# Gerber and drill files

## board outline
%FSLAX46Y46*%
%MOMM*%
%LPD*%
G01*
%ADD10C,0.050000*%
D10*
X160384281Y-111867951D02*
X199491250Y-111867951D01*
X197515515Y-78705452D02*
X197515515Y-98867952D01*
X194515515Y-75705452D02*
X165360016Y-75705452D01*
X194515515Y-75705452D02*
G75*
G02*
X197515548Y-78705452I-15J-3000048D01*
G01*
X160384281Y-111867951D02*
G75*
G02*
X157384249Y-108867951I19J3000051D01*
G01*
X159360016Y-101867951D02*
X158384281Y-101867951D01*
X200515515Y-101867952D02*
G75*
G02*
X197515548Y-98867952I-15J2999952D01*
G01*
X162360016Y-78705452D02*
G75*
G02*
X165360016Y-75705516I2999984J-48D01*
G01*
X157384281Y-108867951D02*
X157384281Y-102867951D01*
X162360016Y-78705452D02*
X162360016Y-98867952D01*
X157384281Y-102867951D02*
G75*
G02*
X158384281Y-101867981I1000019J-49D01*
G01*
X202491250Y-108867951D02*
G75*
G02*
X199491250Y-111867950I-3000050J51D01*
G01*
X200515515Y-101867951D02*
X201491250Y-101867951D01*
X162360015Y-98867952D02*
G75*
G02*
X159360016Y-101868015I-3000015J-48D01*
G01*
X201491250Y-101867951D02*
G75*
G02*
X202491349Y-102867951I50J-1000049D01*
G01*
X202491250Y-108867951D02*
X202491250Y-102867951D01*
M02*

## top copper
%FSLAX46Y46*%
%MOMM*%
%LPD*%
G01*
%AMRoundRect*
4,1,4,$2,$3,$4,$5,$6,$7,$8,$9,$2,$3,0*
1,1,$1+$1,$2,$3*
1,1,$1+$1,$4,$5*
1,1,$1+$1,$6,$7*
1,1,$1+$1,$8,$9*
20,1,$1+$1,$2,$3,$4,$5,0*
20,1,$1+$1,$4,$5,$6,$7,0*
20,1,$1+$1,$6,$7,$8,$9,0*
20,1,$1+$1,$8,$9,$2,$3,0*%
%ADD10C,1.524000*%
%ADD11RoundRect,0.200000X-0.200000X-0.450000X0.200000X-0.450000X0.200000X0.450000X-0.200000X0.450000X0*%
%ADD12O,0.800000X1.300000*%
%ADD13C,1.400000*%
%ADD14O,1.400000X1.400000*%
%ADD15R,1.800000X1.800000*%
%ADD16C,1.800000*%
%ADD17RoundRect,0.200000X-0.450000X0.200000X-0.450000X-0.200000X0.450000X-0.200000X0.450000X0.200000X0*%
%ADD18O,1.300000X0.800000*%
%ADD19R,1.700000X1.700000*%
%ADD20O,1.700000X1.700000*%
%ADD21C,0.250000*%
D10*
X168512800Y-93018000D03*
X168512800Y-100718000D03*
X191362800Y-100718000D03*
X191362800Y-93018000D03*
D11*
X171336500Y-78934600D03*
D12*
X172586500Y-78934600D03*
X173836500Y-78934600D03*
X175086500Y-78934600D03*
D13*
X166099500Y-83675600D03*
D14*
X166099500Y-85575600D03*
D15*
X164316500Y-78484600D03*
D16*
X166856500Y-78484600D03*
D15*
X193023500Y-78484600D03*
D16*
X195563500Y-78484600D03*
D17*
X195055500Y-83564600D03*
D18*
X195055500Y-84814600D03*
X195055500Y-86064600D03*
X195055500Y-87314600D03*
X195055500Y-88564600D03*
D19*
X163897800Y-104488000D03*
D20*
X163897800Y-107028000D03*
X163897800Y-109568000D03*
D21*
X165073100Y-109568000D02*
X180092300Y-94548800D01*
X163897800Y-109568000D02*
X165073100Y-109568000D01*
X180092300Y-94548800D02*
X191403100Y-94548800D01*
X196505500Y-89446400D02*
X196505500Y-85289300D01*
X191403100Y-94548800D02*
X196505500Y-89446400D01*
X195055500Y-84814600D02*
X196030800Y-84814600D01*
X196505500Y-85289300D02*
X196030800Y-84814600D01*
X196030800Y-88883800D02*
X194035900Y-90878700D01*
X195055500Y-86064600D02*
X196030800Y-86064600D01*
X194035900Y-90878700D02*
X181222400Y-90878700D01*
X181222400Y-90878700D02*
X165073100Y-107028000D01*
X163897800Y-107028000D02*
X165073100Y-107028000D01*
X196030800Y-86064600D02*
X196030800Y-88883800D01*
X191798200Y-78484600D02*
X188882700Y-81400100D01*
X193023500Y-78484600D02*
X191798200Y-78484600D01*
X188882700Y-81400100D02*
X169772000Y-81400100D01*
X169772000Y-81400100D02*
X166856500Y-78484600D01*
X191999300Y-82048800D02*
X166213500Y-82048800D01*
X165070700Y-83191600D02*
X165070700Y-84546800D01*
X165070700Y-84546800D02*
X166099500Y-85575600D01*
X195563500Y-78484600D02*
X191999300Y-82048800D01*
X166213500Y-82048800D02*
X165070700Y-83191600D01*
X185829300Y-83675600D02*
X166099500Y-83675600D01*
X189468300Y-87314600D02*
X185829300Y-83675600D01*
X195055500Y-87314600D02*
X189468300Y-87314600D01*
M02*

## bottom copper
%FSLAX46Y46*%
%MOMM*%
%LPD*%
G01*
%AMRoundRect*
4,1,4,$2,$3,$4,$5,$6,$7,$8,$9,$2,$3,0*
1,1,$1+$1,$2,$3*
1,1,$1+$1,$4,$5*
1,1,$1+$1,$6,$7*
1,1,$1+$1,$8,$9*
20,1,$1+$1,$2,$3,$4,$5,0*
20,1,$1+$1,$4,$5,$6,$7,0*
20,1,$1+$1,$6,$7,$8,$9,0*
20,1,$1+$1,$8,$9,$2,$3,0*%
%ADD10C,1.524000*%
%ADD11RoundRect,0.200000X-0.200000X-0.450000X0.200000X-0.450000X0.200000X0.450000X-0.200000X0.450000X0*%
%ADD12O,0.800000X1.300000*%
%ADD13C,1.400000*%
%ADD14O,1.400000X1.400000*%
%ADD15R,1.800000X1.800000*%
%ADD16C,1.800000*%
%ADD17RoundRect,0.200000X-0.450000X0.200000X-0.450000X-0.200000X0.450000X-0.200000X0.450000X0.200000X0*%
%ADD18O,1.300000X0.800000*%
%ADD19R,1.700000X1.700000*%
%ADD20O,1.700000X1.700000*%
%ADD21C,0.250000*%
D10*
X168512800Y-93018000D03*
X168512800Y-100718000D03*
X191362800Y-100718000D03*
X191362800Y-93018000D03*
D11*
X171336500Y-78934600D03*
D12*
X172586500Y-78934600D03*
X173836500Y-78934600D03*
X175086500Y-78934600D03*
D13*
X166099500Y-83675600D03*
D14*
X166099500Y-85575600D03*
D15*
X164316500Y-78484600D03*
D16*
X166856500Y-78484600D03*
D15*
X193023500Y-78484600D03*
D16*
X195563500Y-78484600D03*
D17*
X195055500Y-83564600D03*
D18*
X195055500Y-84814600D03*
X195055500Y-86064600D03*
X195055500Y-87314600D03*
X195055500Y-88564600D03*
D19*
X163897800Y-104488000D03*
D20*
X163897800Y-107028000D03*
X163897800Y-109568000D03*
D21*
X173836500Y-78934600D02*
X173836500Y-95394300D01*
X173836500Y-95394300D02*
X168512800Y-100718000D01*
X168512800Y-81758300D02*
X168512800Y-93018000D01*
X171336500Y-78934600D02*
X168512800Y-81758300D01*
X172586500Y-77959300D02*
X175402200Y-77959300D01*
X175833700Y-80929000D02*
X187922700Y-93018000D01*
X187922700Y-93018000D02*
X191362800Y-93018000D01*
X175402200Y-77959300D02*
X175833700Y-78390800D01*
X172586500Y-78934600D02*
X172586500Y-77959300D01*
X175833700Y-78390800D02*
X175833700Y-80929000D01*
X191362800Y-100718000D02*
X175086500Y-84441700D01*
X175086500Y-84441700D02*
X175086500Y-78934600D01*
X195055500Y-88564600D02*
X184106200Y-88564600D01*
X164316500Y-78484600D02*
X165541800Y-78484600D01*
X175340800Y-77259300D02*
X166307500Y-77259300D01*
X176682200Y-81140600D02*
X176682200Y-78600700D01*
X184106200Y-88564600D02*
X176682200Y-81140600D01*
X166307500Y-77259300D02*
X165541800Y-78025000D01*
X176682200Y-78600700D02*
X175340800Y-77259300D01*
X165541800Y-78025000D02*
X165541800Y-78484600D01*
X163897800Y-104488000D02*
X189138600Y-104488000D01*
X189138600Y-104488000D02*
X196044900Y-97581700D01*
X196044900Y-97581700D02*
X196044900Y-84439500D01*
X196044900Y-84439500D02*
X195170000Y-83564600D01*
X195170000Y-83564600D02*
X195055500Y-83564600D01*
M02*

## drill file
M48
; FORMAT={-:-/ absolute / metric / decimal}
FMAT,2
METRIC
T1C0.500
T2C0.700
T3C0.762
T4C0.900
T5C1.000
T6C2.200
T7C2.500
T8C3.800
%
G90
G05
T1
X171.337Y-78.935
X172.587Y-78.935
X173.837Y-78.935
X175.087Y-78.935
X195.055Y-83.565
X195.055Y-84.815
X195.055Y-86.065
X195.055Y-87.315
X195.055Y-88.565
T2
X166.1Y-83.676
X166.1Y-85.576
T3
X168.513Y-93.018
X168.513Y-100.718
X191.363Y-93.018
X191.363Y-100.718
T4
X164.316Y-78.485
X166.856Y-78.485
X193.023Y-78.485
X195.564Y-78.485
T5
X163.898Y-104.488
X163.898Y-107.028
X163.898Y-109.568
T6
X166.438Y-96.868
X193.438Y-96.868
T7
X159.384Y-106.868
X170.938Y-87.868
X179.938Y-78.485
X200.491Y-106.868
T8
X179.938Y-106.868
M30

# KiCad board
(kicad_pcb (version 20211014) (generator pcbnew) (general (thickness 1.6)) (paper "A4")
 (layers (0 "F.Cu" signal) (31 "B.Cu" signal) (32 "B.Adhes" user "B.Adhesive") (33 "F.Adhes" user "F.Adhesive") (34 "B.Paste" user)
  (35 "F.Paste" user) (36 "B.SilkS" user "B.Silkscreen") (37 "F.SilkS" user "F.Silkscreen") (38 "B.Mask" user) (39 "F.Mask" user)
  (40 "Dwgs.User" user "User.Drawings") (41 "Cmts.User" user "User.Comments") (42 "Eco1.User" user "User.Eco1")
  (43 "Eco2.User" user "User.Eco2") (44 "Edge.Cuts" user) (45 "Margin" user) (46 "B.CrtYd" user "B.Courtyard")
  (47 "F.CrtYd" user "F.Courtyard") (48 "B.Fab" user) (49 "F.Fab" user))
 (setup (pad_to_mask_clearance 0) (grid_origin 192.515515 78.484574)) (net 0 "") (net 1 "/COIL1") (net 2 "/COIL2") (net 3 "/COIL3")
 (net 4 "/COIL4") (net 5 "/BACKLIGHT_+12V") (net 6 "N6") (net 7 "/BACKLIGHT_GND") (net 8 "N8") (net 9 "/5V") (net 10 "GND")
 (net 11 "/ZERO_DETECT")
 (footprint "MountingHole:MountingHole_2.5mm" (layer "F.Cu") (at 179.9378 78.4846)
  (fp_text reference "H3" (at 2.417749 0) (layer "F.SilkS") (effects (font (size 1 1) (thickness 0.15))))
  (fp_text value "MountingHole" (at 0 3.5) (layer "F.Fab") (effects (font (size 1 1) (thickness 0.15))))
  (pad "" np_thru_hole circle locked (at 0 0) (size 2.5 2.5) (drill 2.5) (layers *.Cu *.Mask)))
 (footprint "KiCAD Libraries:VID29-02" (layer "F.Cu") (at 180.1028 96.868)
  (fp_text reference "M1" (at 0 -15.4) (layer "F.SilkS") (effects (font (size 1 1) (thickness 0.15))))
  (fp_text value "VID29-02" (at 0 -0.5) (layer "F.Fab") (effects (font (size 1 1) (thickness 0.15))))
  (pad "" np_thru_hole circle locked (at -9.165 -9) (size 2.5 2.5) (drill 2.5) (layers *.Cu *.Mask))
  (pad "" np_thru_hole circle locked (at 13.335 0) (size 2.2 2.2) (drill 2.2) (layers *.Cu *.Mask))
  (pad "" np_thru_hole circle locked (at -0.165 10) (size 3.8 3.8) (drill 3.8) (layers *.Cu *.Mask))
  (pad "" np_thru_hole circle locked (at -13.665 0) (size 2.2 2.2) (drill 2.2) (layers *.Cu *.Mask))
  (pad "1" thru_hole circle locked (at -11.59 -3.85) (size 1.524 1.524) (drill 0.762) (layers *.Cu *.Mask) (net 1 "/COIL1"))
  (pad "2" thru_hole circle locked (at -11.59 3.85) (size 1.524 1.524) (drill 0.762) (layers *.Cu *.Mask) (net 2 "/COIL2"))
  (pad "3" thru_hole circle locked (at 11.26 3.85) (size 1.524 1.524) (drill 0.762) (layers *.Cu *.Mask) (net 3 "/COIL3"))
  (pad "4" thru_hole circle locked (at 11.26 -3.85) (size 1.524 1.524) (drill 0.762) (layers *.Cu *.Mask) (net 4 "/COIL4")))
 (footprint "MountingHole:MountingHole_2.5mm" (layer "F.Cu") (at 159.3843 106.868)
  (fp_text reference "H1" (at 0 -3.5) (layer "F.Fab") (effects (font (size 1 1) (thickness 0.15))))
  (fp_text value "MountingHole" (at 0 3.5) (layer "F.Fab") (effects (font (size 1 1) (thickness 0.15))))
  (pad "" np_thru_hole circle locked (at 0 0) (size 2.5 2.5) (drill 2.5) (layers *.Cu *.Mask)))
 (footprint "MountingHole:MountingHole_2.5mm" (layer "F.Cu") (at 200.4913 106.868)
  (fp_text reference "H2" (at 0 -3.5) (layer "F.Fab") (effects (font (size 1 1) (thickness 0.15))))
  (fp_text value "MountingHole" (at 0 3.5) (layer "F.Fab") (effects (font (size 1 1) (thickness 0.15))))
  (pad "" np_thru_hole circle locked (at 0 0) (size 2.5 2.5) (drill 2.5) (layers *.Cu *.Mask)))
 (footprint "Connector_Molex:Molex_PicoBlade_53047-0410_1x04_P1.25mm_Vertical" (layer "F.Cu") (at 171.3365 78.9346)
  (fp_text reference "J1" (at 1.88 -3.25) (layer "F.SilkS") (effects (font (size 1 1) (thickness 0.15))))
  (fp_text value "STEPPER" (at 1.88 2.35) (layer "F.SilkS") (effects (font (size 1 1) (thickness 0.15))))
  (pad "1" thru_hole roundrect (at 0 0) (size 0.8 1.3) (drill 0.5) (layers *.Cu *.Mask) (roundrect_rratio 0.25) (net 1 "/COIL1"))
  (pad "2" thru_hole oval (at 1.25 0) (size 0.8 1.3) (drill 0.5) (layers *.Cu *.Mask) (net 4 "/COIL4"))
  (pad "3" thru_hole oval (at 2.5 0) (size 0.8 1.3) (drill 0.5) (layers *.Cu *.Mask) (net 2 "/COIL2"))
  (pad "4" thru_hole oval (at 3.75 0) (size 0.8 1.3) (drill 0.5) (layers *.Cu *.Mask) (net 3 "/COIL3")))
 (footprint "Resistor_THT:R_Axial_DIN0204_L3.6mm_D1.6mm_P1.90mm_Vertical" (layer "F.Cu") (at 166.0995 83.6756 -90)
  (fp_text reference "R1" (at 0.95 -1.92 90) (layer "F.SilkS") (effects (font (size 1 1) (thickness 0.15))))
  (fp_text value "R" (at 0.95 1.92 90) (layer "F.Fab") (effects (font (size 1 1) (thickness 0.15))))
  (pad "1" thru_hole circle (at 0 0 270) (size 1.4 1.4) (drill 0.7) (layers *.Cu *.Mask) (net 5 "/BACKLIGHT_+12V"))
  (pad "2" thru_hole oval (at 1.9 0 270) (size 1.4 1.4) (drill 0.7) (layers *.Cu *.Mask) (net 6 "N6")))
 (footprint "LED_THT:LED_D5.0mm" (layer "F.Cu") (at 164.3165 78.4846)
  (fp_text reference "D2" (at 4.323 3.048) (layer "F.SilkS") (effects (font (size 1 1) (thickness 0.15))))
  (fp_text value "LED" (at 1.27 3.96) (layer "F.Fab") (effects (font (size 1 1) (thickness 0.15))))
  (pad "1" thru_hole rect (at 0 0) (size 1.8 1.8) (drill 0.9) (layers *.Cu *.Mask) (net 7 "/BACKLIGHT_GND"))
  (pad "2" thru_hole circle (at 2.54 0) (size 1.8 1.8) (drill 0.9) (layers *.Cu *.Mask) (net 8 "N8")))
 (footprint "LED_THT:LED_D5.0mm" (layer "F.Cu") (at 193.0235 78.4846)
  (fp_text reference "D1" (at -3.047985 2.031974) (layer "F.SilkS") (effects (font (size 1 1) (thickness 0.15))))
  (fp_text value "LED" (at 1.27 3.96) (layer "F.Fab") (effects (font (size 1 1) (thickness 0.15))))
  (pad "1" thru_hole rect (at 0 0) (size 1.8 1.8) (drill 0.9) (layers *.Cu *.Mask) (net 8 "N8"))
  (pad "2" thru_hole circle (at 2.54 0) (size 1.8 1.8) (drill 0.9) (layers *.Cu *.Mask) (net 6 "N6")))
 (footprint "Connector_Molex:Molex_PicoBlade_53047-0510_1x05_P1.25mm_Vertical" (layer "F.Cu") (at 195.0555 83.5646 -90)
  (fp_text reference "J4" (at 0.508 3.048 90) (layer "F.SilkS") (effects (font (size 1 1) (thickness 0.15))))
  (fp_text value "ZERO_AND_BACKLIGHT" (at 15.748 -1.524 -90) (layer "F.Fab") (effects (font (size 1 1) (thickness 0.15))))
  (pad "1" thru_hole roundrect (at 0 0 270) (size 0.8 1.3) (drill 0.5) (layers *.Cu *.Mask) (roundrect_rratio 0.25) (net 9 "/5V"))
  (pad "2" thru_hole oval (at 1.25 0 270) (size 0.8 1.3) (drill 0.5) (layers *.Cu *.Mask) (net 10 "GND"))
  (pad "3" thru_hole oval (at 2.5 0 270) (size 0.8 1.3) (drill 0.5) (layers *.Cu *.Mask) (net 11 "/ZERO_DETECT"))
  (pad "4" thru_hole oval (at 3.75 0 270) (size 0.8 1.3) (drill 0.5) (layers *.Cu *.Mask) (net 5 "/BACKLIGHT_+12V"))
  (pad "5" thru_hole oval (at 5 0 270) (size 0.8 1.3) (drill 0.5) (layers *.Cu *.Mask) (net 7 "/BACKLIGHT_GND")))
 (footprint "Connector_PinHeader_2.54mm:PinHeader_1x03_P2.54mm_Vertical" (layer "B.Cu") (at 163.8978 104.488 180)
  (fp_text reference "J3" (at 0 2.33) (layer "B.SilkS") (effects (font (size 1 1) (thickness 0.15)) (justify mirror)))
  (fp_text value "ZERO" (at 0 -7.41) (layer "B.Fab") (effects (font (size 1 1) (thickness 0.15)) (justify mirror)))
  (pad "1" thru_hole rect locked (at 0 0 180) (size 1.7 1.7) (drill 1) (layers *.Cu *.Mask) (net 9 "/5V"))
  (pad "2" thru_hole oval locked (at 0 -2.54 180) (size 1.7 1.7) (drill 1) (layers *.Cu *.Mask) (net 11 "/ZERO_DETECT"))
  (pad "3" thru_hole oval locked (at 0 -5.08 180) (size 1.7 1.7) (drill 1) (layers *.Cu *.Mask) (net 10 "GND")))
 (gr_line (start 160.384281 111.867951) (end 199.49125 111.867951) (layer "Edge.Cuts") (width 0.05))
 (gr_line (start 197.515515 78.705452) (end 197.515515 98.867952) (layer "Edge.Cuts") (width 0.05))
 (gr_line (start 194.515515 75.705452) (end 165.360016 75.705452) (layer "Edge.Cuts") (width 0.05))
 (gr_arc (start 194.515515 75.705452) (mid 196.636835 76.584132) (end 197.515515 78.705452) (layer "Edge.Cuts") (width 0.05))
 (gr_arc (start 160.384281 111.867951) (mid 158.262961 110.989271) (end 157.384281 108.867951) (layer "Edge.Cuts") (width 0.05))
 (gr_line (start 159.360016 101.867951) (end 158.384281 101.867951) (layer "Edge.Cuts") (width 0.05))
 (gr_arc (start 200.515515 101.867952) (mid 198.394195 100.989272) (end 197.515515 98.867952) (layer "Edge.Cuts") (width 0.05))
 (gr_arc (start 162.360016 78.705452) (mid 163.238696 76.584132) (end 165.360016 75.705452) (layer "Edge.Cuts") (width 0.05))
 (gr_line (start 157.384281 108.867951) (end 157.384281 102.867951) (layer "Edge.Cuts") (width 0.05))
 (gr_line (start 162.360016 78.705452) (end 162.360016 98.867952) (layer "Edge.Cuts") (width 0.05))
 (gr_arc (start 157.384281 102.867951) (mid 157.677174 102.160844) (end 158.384281 101.867951) (layer "Edge.Cuts") (width 0.05))
 (gr_arc (start 202.49125 108.867951) (mid 201.61257 110.989271) (end 199.49125 111.867951) (layer "Edge.Cuts") (width 0.05))
 (gr_line (start 200.515515 101.867951) (end 201.49125 101.867951) (layer "Edge.Cuts") (width 0.05))
 (gr_arc (start 162.360015 98.867952) (mid 161.481336 100.989272) (end 159.360016 101.867951) (layer "Edge.Cuts") (width 0.05))
 (gr_arc (start 201.49125 101.867951) (mid 202.198357 102.160844) (end 202.49125 102.867951) (layer "Edge.Cuts") (width 0.05))
 (gr_line (start 202.49125 108.867951) (end 202.49125 102.867951) (layer "Edge.Cuts") (width 0.05))
 (segment (start 165.0731 109.568) (end 180.0923 94.5488) (width 0.25) (layer "F.Cu") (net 10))
 (segment (start 163.8978 109.568) (end 165.0731 109.568) (width 0.25) (layer "F.Cu") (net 10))
 (segment (start 180.0923 94.5488) (end 191.4031 94.5488) (width 0.25) (layer "F.Cu") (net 10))
 (segment (start 196.5055 89.4464) (end 196.5055 85.2893) (width 0.25) (layer "F.Cu") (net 10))
 (segment (start 191.4031 94.5488) (end 196.5055 89.4464) (width 0.25) (layer "F.Cu") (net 10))
 (segment (start 195.0555 84.8146) (end 196.0308 84.8146) (width 0.25) (layer "F.Cu") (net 10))
 (segment (start 196.5055 85.2893) (end 196.0308 84.8146) (width 0.25) (layer "F.Cu") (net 10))
 (segment (start 196.0308 88.8838) (end 194.0359 90.8787) (width 0.25) (layer "F.Cu") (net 11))
 (segment (start 195.0555 86.0646) (end 196.0308 86.0646) (width 0.25) (layer "F.Cu") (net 11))
 (segment (start 194.0359 90.8787) (end 181.2224 90.8787) (width 0.25) (layer "F.Cu") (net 11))
 (segment (start 181.2224 90.8787) (end 165.0731 107.028) (width 0.25) (layer "F.Cu") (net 11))
 (segment (start 163.8978 107.028) (end 165.0731 107.028) (width 0.25) (layer "F.Cu") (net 11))
 (segment (start 196.0308 86.0646) (end 196.0308 88.8838) (width 0.25) (layer "F.Cu") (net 11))
 (segment (start 173.8365 78.9346) (end 173.8365 95.3943) (width 0.25) (layer "B.Cu") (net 2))
 (segment (start 173.8365 95.3943) (end 168.5128 100.718) (width 0.25) (layer "B.Cu") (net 2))
 (segment (start 168.5128 81.7583) (end 168.5128 93.018) (width 0.25) (layer "B.Cu") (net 1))
 (segment (start 171.3365 78.9346) (end 168.5128 81.7583) (width 0.25) (layer "B.Cu") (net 1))
 (segment (start 172.5865 77.9593) (end 175.4022 77.9593) (width 0.25) (layer "B.Cu") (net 4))
 (segment (start 175.8337 80.929) (end 187.9227 93.018) (width 0.25) (layer "B.Cu") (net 4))
 (segment (start 187.9227 93.018) (end 191.3628 93.018) (width 0.25) (layer "B.Cu") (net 4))
 (segment (start 175.4022 77.9593) (end 175.8337 78.3908) (width 0.25) (layer "B.Cu") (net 4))
 (segment (start 172.5865 78.9346) (end 172.5865 77.9593) (width 0.25) (layer "B.Cu") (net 4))
 (segment (start 175.8337 78.3908) (end 175.8337 80.929) (width 0.25) (layer "B.Cu") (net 4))
 (segment (start 191.3628 100.718) (end 175.0865 84.4417) (width 0.25) (layer "B.Cu") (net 3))
 (segment (start 175.0865 84.4417) (end 175.0865 78.9346) (width 0.25) (layer "B.Cu") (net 3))
 (segment (start 191.7982 78.4846) (end 188.8827 81.4001) (width 0.25) (layer "F.Cu") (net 8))
 (segment (start 193.0235 78.4846) (end 191.7982 78.4846) (width 0.25) (layer "F.Cu") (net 8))
 (segment (start 188.8827 81.4001) (end 169.772 81.4001) (width 0.25) (layer "F.Cu") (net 8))
 (segment (start 169.772 81.4001) (end 166.8565 78.4846) (width 0.25) (layer "F.Cu") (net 8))
 (segment (start 191.9993 82.0488) (end 166.2135 82.0488) (width 0.25) (layer "F.Cu") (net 6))
 (segment (start 165.0707 83.1916) (end 165.0707 84.5468) (width 0.25) (layer "F.Cu") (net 6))
 (segment (start 165.0707 84.5468) (end 166.0995 85.5756) (width 0.25) (layer "F.Cu") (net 6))
 (segment (start 195.5635 78.4846) (end 191.9993 82.0488) (width 0.25) (layer "F.Cu") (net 6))
 (segment (start 166.2135 82.0488) (end 165.0707 83.1916) (width 0.25) (layer "F.Cu") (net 6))
 (segment (start 195.0555 88.5646) (end 184.1062 88.5646) (width 0.25) (layer "B.Cu") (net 7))
 (segment (start 164.3165 78.4846) (end 165.5418 78.4846) (width 0.25) (layer "B.Cu") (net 7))
 (segment (start 175.3408 77.2593) (end 166.3075 77.2593) (width 0.25) (layer "B.Cu") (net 7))
 (segment (start 176.6822 81.1406) (end 176.6822 78.6007) (width 0.25) (layer "B.Cu") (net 7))
 (segment (start 184.1062 88.5646) (end 176.6822 81.1406) (width 0.25) (layer "B.Cu") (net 7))
 (segment (start 166.3075 77.2593) (end 165.5418 78.025) (width 0.25) (layer "B.Cu") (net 7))
 (segment (start 176.6822 78.6007) (end 175.3408 77.2593) (width 0.25) (layer "B.Cu") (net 7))
 (segment (start 165.5418 78.025) (end 165.5418 78.4846) (width 0.25) (layer "B.Cu") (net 7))
 (segment (start 185.8293 83.6756) (end 166.0995 83.6756) (width 0.25) (layer "F.Cu") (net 5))
 (segment (start 189.4683 87.3146) (end 185.8293 83.6756) (width 0.25) (layer "F.Cu") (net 5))
 (segment (start 195.0555 87.3146) (end 189.4683 87.3146) (width 0.25) (layer "F.Cu") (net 5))
 (segment (start 163.8978 104.488) (end 189.1386 104.488) (width 0.25) (layer "B.Cu") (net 9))
 (segment (start 189.1386 104.488) (end 196.0449 97.5817) (width 0.25) (layer "B.Cu") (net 9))
 (segment (start 196.0449 97.5817) (end 196.0449 84.4395) (width 0.25) (layer "B.Cu") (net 9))
 (segment (start 196.0449 84.4395) (end 195.17 83.5646) (width 0.25) (layer "B.Cu") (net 9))
 (segment (start 195.17 83.5646) (end 195.0555 83.5646) (width 0.25) (layer "B.Cu") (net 9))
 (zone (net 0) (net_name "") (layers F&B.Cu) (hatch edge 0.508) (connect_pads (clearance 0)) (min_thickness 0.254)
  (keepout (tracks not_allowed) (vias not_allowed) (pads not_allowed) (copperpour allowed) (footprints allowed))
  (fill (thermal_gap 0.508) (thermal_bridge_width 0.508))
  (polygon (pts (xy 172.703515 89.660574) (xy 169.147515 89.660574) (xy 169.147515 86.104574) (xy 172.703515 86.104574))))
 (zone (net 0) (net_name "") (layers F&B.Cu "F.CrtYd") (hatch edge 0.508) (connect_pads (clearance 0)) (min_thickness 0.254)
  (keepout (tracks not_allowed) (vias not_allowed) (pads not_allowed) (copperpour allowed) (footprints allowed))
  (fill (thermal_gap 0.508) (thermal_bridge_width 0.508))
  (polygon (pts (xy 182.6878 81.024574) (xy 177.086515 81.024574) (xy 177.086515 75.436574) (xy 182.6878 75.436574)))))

